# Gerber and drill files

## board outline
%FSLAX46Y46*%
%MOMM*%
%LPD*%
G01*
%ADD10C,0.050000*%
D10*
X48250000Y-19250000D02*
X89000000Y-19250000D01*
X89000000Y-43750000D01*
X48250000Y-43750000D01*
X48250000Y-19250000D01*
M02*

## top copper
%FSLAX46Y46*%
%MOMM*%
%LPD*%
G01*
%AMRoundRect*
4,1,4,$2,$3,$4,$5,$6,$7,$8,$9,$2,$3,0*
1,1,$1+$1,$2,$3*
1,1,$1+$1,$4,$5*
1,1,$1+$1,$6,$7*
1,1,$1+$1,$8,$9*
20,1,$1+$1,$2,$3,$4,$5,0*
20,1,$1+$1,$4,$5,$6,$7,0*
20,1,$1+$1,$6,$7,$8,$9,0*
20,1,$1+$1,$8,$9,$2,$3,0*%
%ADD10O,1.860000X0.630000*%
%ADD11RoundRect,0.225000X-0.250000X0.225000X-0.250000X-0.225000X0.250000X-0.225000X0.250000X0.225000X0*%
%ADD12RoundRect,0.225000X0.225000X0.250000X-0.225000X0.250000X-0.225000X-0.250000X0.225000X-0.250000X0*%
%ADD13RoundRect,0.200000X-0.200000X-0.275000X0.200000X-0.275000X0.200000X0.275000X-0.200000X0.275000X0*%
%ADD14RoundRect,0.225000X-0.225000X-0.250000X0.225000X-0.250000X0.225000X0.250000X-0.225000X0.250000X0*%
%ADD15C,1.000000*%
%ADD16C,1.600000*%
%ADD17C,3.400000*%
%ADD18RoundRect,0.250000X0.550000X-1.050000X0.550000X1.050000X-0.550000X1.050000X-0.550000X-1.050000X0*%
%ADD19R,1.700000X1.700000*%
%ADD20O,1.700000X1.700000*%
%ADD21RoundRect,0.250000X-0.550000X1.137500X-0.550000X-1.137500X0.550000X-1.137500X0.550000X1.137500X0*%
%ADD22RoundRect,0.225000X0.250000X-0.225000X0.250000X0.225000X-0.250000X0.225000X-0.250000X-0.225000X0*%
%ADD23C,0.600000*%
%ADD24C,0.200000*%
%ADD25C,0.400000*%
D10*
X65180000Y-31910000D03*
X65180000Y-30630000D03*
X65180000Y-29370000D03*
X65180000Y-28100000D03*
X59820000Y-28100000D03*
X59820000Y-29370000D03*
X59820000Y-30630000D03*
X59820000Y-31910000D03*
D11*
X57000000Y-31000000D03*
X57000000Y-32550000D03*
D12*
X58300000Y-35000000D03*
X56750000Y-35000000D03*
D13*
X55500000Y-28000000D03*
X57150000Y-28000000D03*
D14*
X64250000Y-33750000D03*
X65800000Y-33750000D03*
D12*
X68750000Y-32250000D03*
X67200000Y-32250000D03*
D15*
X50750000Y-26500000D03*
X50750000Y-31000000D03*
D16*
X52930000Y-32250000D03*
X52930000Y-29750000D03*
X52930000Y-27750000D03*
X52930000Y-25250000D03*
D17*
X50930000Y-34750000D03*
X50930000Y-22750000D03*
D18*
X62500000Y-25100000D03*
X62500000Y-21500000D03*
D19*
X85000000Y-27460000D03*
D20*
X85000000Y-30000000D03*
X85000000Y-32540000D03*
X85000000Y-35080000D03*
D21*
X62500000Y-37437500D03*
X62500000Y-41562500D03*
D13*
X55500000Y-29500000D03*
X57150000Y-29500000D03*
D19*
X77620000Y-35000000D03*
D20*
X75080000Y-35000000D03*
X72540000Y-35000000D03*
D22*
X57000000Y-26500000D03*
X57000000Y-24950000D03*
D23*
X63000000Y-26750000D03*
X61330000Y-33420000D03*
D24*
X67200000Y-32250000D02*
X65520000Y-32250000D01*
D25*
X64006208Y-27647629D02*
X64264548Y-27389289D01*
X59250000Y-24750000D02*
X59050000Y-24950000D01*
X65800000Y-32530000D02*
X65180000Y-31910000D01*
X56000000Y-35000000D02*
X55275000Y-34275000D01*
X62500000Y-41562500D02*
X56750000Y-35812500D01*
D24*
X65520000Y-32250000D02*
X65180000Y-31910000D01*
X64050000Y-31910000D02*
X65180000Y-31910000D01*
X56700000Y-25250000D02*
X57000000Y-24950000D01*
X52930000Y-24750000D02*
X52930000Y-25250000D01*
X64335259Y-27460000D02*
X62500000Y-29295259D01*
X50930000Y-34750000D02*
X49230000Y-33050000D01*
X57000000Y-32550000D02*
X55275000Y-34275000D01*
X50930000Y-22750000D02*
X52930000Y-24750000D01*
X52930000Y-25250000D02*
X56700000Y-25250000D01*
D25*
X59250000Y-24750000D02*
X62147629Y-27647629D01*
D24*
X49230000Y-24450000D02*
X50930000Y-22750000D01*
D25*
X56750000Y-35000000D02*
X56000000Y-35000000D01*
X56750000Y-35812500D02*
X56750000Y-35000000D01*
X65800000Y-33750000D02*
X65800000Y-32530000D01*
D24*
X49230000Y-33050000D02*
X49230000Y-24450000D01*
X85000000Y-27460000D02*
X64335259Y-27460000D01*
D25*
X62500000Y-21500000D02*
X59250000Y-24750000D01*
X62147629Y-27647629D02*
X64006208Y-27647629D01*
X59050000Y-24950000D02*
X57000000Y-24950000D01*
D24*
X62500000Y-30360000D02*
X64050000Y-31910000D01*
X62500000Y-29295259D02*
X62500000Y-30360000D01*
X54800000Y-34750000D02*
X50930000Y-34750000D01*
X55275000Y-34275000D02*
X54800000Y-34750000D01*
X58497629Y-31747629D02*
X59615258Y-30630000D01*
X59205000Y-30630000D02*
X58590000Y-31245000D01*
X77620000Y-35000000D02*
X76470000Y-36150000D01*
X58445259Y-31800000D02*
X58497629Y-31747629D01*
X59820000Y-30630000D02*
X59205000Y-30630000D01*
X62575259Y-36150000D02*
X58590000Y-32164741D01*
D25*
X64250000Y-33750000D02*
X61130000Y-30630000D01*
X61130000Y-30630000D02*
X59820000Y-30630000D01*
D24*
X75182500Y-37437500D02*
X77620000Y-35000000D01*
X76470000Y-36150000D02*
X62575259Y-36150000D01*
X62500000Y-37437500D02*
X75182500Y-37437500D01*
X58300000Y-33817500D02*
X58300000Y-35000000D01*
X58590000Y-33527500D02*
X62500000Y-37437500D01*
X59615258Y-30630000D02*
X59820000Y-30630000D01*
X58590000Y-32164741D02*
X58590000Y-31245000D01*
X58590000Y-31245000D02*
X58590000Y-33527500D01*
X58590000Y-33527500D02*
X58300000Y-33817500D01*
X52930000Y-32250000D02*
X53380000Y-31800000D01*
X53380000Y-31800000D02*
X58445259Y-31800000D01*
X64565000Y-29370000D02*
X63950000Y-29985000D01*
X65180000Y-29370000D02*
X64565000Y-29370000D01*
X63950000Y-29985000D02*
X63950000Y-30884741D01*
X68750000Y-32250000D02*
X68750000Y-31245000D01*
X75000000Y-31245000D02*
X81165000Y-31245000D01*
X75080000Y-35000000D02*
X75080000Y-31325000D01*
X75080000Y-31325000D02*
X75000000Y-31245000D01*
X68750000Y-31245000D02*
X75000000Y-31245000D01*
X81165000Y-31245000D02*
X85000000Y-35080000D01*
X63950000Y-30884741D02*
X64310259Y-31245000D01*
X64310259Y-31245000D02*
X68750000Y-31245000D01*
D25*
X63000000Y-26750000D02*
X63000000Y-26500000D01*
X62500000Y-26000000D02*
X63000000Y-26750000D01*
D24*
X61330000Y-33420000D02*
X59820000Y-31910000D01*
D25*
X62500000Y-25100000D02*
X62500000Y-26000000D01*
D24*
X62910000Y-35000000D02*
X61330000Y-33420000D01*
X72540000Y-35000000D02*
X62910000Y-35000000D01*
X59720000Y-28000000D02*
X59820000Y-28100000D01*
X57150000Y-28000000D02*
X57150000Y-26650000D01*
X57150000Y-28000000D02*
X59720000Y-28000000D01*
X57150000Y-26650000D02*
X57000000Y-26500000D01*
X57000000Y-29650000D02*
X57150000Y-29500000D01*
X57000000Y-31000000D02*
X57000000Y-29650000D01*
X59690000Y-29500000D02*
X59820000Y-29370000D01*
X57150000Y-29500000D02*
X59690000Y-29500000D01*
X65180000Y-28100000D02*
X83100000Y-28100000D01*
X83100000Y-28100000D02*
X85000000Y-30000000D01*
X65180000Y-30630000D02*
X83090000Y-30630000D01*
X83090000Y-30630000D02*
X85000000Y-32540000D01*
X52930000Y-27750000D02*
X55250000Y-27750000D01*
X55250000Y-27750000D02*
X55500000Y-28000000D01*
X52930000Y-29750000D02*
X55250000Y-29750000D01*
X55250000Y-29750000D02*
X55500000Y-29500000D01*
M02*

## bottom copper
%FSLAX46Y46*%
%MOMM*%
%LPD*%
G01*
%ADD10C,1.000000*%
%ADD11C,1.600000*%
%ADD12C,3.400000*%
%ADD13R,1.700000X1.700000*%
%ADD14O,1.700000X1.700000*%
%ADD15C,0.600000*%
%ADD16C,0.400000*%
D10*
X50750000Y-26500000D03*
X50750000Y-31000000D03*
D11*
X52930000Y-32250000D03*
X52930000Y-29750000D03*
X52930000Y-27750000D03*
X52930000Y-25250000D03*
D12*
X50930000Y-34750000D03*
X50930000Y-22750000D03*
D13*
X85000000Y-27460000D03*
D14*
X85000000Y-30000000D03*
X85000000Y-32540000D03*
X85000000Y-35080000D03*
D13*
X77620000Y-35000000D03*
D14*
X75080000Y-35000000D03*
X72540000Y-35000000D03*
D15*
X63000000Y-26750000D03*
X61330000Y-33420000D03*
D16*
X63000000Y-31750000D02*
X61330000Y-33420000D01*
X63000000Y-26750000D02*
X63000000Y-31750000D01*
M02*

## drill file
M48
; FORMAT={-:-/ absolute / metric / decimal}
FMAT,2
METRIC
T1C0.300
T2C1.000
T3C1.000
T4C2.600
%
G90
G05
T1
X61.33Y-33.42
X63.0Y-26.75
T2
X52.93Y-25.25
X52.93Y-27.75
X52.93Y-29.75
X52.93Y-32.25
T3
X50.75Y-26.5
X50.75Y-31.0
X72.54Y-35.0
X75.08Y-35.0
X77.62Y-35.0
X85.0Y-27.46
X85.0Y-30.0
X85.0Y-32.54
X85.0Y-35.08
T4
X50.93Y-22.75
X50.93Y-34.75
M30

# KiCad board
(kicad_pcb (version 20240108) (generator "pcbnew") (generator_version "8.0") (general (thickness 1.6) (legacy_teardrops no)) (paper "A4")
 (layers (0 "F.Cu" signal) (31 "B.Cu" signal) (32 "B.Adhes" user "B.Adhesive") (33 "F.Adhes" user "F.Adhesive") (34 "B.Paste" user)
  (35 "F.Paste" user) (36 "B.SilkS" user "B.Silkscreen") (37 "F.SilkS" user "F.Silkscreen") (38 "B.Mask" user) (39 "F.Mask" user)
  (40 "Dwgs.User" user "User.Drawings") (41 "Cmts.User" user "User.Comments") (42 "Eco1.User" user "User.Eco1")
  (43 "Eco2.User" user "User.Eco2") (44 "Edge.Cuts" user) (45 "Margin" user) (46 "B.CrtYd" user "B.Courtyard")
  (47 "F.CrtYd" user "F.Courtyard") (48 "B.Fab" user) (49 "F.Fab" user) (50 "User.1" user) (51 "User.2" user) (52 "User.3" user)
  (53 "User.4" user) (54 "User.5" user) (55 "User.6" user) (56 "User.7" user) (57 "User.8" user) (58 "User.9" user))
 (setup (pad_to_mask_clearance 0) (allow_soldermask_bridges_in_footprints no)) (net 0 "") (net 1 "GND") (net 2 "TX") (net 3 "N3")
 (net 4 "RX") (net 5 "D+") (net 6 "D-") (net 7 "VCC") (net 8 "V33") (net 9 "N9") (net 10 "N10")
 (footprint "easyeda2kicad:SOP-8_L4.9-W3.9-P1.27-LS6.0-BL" (layer "F.Cu") (at 62.5 30 90)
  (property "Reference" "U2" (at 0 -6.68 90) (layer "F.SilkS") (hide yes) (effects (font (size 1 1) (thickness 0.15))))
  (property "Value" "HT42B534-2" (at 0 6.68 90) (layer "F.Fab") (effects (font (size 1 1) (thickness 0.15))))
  (pad "1" smd oval (at -1.91 2.68 90) (size 0.63 1.86) (layers "F.Cu" "F.Paste" "F.Mask") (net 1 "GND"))
  (pad "2" smd oval (at -0.63 2.68 90) (size 0.63 1.86) (layers "F.Cu" "F.Paste" "F.Mask") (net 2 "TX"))
  (pad "3" smd oval (at 0.63 2.68 90) (size 0.63 1.86) (layers "F.Cu" "F.Paste" "F.Mask") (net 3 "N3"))
  (pad "4" smd oval (at 1.9 2.68 90) (size 0.63 1.86) (layers "F.Cu" "F.Paste" "F.Mask") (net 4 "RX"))
  (pad "5" smd oval (at 1.9 -2.68 90) (size 0.63 1.86) (layers "F.Cu" "F.Paste" "F.Mask") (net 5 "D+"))
  (pad "6" smd oval (at 0.63 -2.68 90) (size 0.63 1.86) (layers "F.Cu" "F.Paste" "F.Mask") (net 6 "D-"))
  (pad "7" smd oval (at -0.63 -2.68 90) (size 0.63 1.86) (layers "F.Cu" "F.Paste" "F.Mask") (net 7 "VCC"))
  (pad "8" smd oval (at -1.91 -2.68 90) (size 0.63 1.86) (layers "F.Cu" "F.Paste" "F.Mask") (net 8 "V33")))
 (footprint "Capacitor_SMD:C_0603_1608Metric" (layer "F.Cu") (at 57 31.775 -90)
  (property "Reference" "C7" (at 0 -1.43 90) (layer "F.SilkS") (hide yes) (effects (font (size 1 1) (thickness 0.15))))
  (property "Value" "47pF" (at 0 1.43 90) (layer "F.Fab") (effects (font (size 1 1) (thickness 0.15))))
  (pad "1" smd roundrect (at -0.775 0 270) (size 0.9 0.95) (layers "F.Cu" "F.Paste" "F.Mask") (roundrect_rratio 0.25) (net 6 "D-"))
  (pad "2" smd roundrect (at 0.775 0 270) (size 0.9 0.95) (layers "F.Cu" "F.Paste" "F.Mask") (roundrect_rratio 0.25) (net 1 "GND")))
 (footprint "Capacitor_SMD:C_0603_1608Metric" (layer "F.Cu") (at 57.525 35 180)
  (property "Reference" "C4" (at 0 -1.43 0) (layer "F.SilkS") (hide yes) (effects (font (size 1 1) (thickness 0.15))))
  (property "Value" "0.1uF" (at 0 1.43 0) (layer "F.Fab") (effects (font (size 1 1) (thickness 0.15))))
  (pad "1" smd roundrect (at -0.775 0 180) (size 0.9 0.95) (layers "F.Cu" "F.Paste" "F.Mask") (roundrect_rratio 0.25) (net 7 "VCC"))
  (pad "2" smd roundrect (at 0.775 0 180) (size 0.9 0.95) (layers "F.Cu" "F.Paste" "F.Mask") (roundrect_rratio 0.25) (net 1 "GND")))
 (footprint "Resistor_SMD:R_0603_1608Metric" (layer "F.Cu") (at 56.325 28)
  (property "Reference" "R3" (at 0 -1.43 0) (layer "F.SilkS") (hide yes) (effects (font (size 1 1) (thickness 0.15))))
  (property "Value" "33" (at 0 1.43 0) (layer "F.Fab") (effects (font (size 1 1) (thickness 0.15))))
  (pad "1" smd roundrect (at -0.825 0) (size 0.8 0.95) (layers "F.Cu" "F.Paste" "F.Mask") (roundrect_rratio 0.25) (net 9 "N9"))
  (pad "2" smd roundrect (at 0.825 0) (size 0.8 0.95) (layers "F.Cu" "F.Paste" "F.Mask") (roundrect_rratio 0.25) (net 5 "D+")))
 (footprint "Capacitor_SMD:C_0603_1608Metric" (layer "F.Cu") (at 65.025 33.75)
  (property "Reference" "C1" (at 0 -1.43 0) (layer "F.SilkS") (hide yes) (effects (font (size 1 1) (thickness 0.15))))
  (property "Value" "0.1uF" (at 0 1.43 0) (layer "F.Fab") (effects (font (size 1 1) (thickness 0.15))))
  (pad "1" smd roundrect (at -0.775 0) (size 0.9 0.95) (layers "F.Cu" "F.Paste" "F.Mask") (roundrect_rratio 0.25) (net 7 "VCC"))
  (pad "2" smd roundrect (at 0.775 0) (size 0.9 0.95) (layers "F.Cu" "F.Paste" "F.Mask") (roundrect_rratio 0.25) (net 1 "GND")))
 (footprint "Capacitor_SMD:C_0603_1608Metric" (layer "F.Cu") (at 67.975 32.25 180)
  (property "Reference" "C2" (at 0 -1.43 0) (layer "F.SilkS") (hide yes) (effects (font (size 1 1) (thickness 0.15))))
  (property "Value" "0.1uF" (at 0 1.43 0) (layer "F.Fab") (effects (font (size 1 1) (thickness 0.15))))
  (pad "1" smd roundrect (at -0.775 0 180) (size 0.9 0.95) (layers "F.Cu" "F.Paste" "F.Mask") (roundrect_rratio 0.25) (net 3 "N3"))
  (pad "2" smd roundrect (at 0.775 0 180) (size 0.9 0.95) (layers "F.Cu" "F.Paste" "F.Mask") (roundrect_rratio 0.25) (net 1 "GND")))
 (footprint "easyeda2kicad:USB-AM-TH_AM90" (layer "F.Cu") (at 51.93 28.75 -90)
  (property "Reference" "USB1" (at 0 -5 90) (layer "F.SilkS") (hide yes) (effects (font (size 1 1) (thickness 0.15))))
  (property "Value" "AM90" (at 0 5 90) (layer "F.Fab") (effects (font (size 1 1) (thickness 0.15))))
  (pad "" thru_hole circle (at -2.25 1.18 270) (size 1 1) (drill 1) (layers "*.Cu" "*.Mask") (remove_unused_layers no))
  (pad "" thru_hole circle (at 2.25 1.18 270) (size 1 1) (drill 1) (layers "*.Cu" "*.Mask") (remove_unused_layers no))
  (pad "1" thru_hole circle (at 3.5 -1 180) (size 1.6 1.6) (drill 0.999998) (layers "*.Cu" "*.Mask") (remove_unused_layers no) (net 7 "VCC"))
  (pad "2" thru_hole circle (at 1 -1 180) (size 1.6 1.6) (drill 0.999998) (layers "*.Cu" "*.Mask") (remove_unused_layers no) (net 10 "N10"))
  (pad "3" thru_hole circle (at -1 -1 180) (size 1.6 1.6) (drill 0.999998) (layers "*.Cu" "*.Mask") (remove_unused_layers no) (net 9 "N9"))
  (pad "4" thru_hole circle (at -3.5 -1 180) (size 1.6 1.6) (drill 0.999998) (layers "*.Cu" "*.Mask") (remove_unused_layers no)
   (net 1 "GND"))
  (pad "MH1" thru_hole circle (at 6 1 180) (size 3.4 3.4) (drill 2.599995) (layers "*.Cu" "*.Mask") (remove_unused_layers no) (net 1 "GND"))
  (pad "MH2" thru_hole circle (at -6 1 180) (size 3.4 3.4) (drill 2.599995) (layers "*.Cu" "*.Mask") (remove_unused_layers no) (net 1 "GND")))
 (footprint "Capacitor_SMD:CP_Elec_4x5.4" (layer "F.Cu") (at 62.5 23.3 90)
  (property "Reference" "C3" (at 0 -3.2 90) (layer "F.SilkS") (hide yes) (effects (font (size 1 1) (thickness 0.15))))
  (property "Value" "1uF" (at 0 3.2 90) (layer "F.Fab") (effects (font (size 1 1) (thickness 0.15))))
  (pad "1" smd roundrect (at -1.8 0 90) (size 2.6 1.6) (layers "F.Cu" "F.Paste" "F.Mask") (roundrect_rratio 0.15625) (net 8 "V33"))
  (pad "2" smd roundrect (at 1.8 0 90) (size 2.6 1.6) (layers "F.Cu" "F.Paste" "F.Mask") (roundrect_rratio 0.15625) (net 1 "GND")))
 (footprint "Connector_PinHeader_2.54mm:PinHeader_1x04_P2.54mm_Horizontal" (layer "F.Cu") (at 85 27.46)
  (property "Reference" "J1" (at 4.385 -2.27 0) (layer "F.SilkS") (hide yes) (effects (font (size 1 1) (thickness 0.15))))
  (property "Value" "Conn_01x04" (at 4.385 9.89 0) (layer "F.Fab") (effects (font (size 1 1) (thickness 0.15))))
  (pad "1" thru_hole rect (at 0 0) (size 1.7 1.7) (drill 1) (layers "*.Cu" "*.Mask") (remove_unused_layers no) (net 1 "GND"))
  (pad "2" thru_hole oval (at 0 2.54) (size 1.7 1.7) (drill 1) (layers "*.Cu" "*.Mask") (remove_unused_layers no) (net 4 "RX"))
  (pad "3" thru_hole oval (at 0 5.08) (size 1.7 1.7) (drill 1) (layers "*.Cu" "*.Mask") (remove_unused_layers no) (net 2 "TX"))
  (pad "4" thru_hole oval (at 0 7.62) (size 1.7 1.7) (drill 1) (layers "*.Cu" "*.Mask") (remove_unused_layers no) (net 3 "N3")))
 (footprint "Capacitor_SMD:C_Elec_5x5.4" (layer "F.Cu") (at 62.5 39.5 -90)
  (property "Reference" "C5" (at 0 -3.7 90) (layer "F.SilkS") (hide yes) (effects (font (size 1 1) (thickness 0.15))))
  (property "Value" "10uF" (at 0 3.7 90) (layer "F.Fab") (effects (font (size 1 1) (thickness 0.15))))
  (pad "1" smd roundrect (at -2.0625 0 270) (size 2.775 1.6) (layers "F.Cu" "F.Paste" "F.Mask") (roundrect_rratio 0.15625) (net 7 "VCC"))
  (pad "2" smd roundrect (at 2.0625 0 270) (size 2.775 1.6) (layers "F.Cu" "F.Paste" "F.Mask") (roundrect_rratio 0.15625) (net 1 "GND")))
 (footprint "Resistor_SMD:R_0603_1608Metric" (layer "F.Cu") (at 56.325 29.5)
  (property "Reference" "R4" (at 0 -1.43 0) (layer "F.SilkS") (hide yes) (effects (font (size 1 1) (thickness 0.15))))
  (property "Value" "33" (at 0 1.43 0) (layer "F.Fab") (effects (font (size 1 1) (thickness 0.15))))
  (pad "1" smd roundrect (at -0.825 0) (size 0.8 0.95) (layers "F.Cu" "F.Paste" "F.Mask") (roundrect_rratio 0.25) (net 10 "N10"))
  (pad "2" smd roundrect (at 0.825 0) (size 0.8 0.95) (layers "F.Cu" "F.Paste" "F.Mask") (roundrect_rratio 0.25) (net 6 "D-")))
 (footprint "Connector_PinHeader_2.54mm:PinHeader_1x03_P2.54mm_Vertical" (layer "F.Cu") (at 77.62 35 -90)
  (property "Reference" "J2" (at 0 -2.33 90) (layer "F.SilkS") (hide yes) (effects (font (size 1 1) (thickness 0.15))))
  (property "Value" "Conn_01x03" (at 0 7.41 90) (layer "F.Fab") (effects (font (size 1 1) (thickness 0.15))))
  (pad "1" thru_hole rect (at 0 0 270) (size 1.7 1.7) (drill 1) (layers "*.Cu" "*.Mask") (remove_unused_layers no) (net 7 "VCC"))
  (pad "2" thru_hole oval (at 0 2.54 270) (size 1.7 1.7) (drill 1) (layers "*.Cu" "*.Mask") (remove_unused_layers no) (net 3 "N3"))
  (pad "3" thru_hole oval (at 0 5.08 270) (size 1.7 1.7) (drill 1) (layers "*.Cu" "*.Mask") (remove_unused_layers no) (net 8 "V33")))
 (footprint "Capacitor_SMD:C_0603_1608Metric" (layer "F.Cu") (at 57 25.725 90)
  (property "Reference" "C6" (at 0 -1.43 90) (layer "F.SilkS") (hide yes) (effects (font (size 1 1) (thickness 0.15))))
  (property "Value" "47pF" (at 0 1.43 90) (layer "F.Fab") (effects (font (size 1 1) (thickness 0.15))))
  (pad "1" smd roundrect (at -0.775 0 90) (size 0.9 0.95) (layers "F.Cu" "F.Paste" "F.Mask") (roundrect_rratio 0.25) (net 5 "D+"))
  (pad "2" smd roundrect (at 0.775 0 90) (size 0.9 0.95) (layers "F.Cu" "F.Paste" "F.Mask") (roundrect_rratio 0.25) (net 1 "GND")))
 (gr_rect (start 48.25 19.25) (end 89 43.75) (stroke (width 0.05) (type default)) (fill none) (layer "Edge.Cuts"))
 (segment (start 67.2 32.25) (end 65.52 32.25) (width 0.2) (layer "F.Cu") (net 1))
 (segment (start 64.006208 27.647629) (end 64.264548 27.389289) (width 0.4) (layer "F.Cu") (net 1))
 (segment (start 59.25 24.75) (end 59.05 24.95) (width 0.4) (layer "F.Cu") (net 1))
 (segment (start 65.8 32.53) (end 65.18 31.91) (width 0.4) (layer "F.Cu") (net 1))
 (segment (start 56 35) (end 55.275 34.275) (width 0.4) (layer "F.Cu") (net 1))
 (segment (start 62.5 41.5625) (end 56.75 35.8125) (width 0.4) (layer "F.Cu") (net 1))
 (segment (start 65.52 32.25) (end 65.18 31.91) (width 0.2) (layer "F.Cu") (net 1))
 (segment (start 64.05 31.91) (end 65.18 31.91) (width 0.2) (layer "F.Cu") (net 1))
 (segment (start 56.7 25.25) (end 57 24.95) (width 0.2) (layer "F.Cu") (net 1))
 (segment (start 52.93 24.75) (end 52.93 25.25) (width 0.2) (layer "F.Cu") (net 1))
 (segment (start 64.335259 27.46) (end 62.5 29.295259) (width 0.2) (layer "F.Cu") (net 1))
 (segment (start 50.93 34.75) (end 49.23 33.05) (width 0.2) (layer "F.Cu") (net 1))
 (segment (start 57 32.55) (end 55.275 34.275) (width 0.2) (layer "F.Cu") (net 1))
 (segment (start 50.93 22.75) (end 52.93 24.75) (width 0.2) (layer "F.Cu") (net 1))
 (segment (start 52.93 25.25) (end 56.7 25.25) (width 0.2) (layer "F.Cu") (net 1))
 (segment (start 59.25 24.75) (end 62.147629 27.647629) (width 0.4) (layer "F.Cu") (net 1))
 (segment (start 49.23 24.45) (end 50.93 22.75) (width 0.2) (layer "F.Cu") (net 1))
 (segment (start 56.75 35) (end 56 35) (width 0.4) (layer "F.Cu") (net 1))
 (segment (start 56.75 35.8125) (end 56.75 35) (width 0.4) (layer "F.Cu") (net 1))
 (segment (start 65.8 33.75) (end 65.8 32.53) (width 0.4) (layer "F.Cu") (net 1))
 (segment (start 49.23 33.05) (end 49.23 24.45) (width 0.2) (layer "F.Cu") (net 1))
 (segment (start 85 27.46) (end 64.335259 27.46) (width 0.2) (layer "F.Cu") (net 1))
 (segment (start 62.5 21.5) (end 59.25 24.75) (width 0.4) (layer "F.Cu") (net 1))
 (segment (start 62.147629 27.647629) (end 64.006208 27.647629) (width 0.4) (layer "F.Cu") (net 1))
 (segment (start 59.05 24.95) (end 57 24.95) (width 0.4) (layer "F.Cu") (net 1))
 (segment (start 62.5 30.36) (end 64.05 31.91) (width 0.2) (layer "F.Cu") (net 1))
 (segment (start 62.5 29.295259) (end 62.5 30.36) (width 0.2) (layer "F.Cu") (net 1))
 (segment (start 54.8 34.75) (end 50.93 34.75) (width 0.2) (layer "F.Cu") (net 1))
 (segment (start 55.275 34.275) (end 54.8 34.75) (width 0.2) (layer "F.Cu") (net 1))
 (segment (start 58.497629 31.747629) (end 59.615258 30.63) (width 0.2) (layer "F.Cu") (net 7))
 (segment (start 59.205 30.63) (end 58.59 31.245) (width 0.2) (layer "F.Cu") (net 7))
 (segment (start 77.62 35) (end 76.47 36.15) (width 0.2) (layer "F.Cu") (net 7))
 (segment (start 58.445259 31.8) (end 58.497629 31.747629) (width 0.2) (layer "F.Cu") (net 7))
 (segment (start 59.82 30.63) (end 59.205 30.63) (width 0.2) (layer "F.Cu") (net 7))
 (segment (start 62.575259 36.15) (end 58.59 32.164741) (width 0.2) (layer "F.Cu") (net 7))
 (segment (start 64.25 33.75) (end 61.13 30.63) (width 0.4) (layer "F.Cu") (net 7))
 (segment (start 61.13 30.63) (end 59.82 30.63) (width 0.4) (layer "F.Cu") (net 7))
 (segment (start 75.1825 37.4375) (end 77.62 35) (width 0.2) (layer "F.Cu") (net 7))
 (segment (start 76.47 36.15) (end 62.575259 36.15) (width 0.2) (layer "F.Cu") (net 7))
 (segment (start 62.5 37.4375) (end 75.1825 37.4375) (width 0.2) (layer "F.Cu") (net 7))
 (segment (start 58.3 33.8175) (end 58.3 35) (width 0.2) (layer "F.Cu") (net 7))
 (segment (start 58.59 33.5275) (end 62.5 37.4375) (width 0.2) (layer "F.Cu") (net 7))
 (segment (start 59.615258 30.63) (end 59.82 30.63) (width 0.2) (layer "F.Cu") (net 7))
 (segment (start 58.59 32.164741) (end 58.59 31.245) (width 0.2) (layer "F.Cu") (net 7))
 (segment (start 58.59 31.245) (end 58.59 33.5275) (width 0.2) (layer "F.Cu") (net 7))
 (segment (start 58.59 33.5275) (end 58.3 33.8175) (width 0.2) (layer "F.Cu") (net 7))
 (segment (start 52.93 32.25) (end 53.38 31.8) (width 0.2) (layer "F.Cu") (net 7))
 (segment (start 53.38 31.8) (end 58.445259 31.8) (width 0.2) (layer "F.Cu") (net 7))
 (segment (start 64.565 29.37) (end 63.95 29.985) (width 0.2) (layer "F.Cu") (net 3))
 (segment (start 65.18 29.37) (end 64.565 29.37) (width 0.2) (layer "F.Cu") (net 3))
 (segment (start 63.95 29.985) (end 63.95 30.884741) (width 0.2) (layer "F.Cu") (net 3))
 (segment (start 68.75 32.25) (end 68.75 31.245) (width 0.2) (layer "F.Cu") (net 3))
 (segment (start 75 31.245) (end 81.165 31.245) (width 0.2) (layer "F.Cu") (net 3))
 (segment (start 75.08 35) (end 75.08 31.325) (width 0.2) (layer "F.Cu") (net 3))
 (segment (start 75.08 31.325) (end 75 31.245) (width 0.2) (layer "F.Cu") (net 3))
 (segment (start 68.75 31.245) (end 75 31.245) (width 0.2) (layer "F.Cu") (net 3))
 (segment (start 81.165 31.245) (end 85 35.08) (width 0.2) (layer "F.Cu") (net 3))
 (segment (start 63.95 30.884741) (end 64.310259 31.245) (width 0.2) (layer "F.Cu") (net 3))
 (segment (start 64.310259 31.245) (end 68.75 31.245) (width 0.2) (layer "F.Cu") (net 3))
 (segment (start 63 26.75) (end 63 26.5) (width 0.4) (layer "F.Cu") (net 8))
 (segment (start 62.5 26) (end 63 26.75) (width 0.4) (layer "F.Cu") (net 8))
 (segment (start 61.33 33.42) (end 59.82 31.91) (width 0.2) (layer "F.Cu") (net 8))
 (segment (start 62.5 25.1) (end 62.5 26) (width 0.4) (layer "F.Cu") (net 8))
 (segment (start 62.91 35) (end 61.33 33.42) (width 0.2) (layer "F.Cu") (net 8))
 (segment (start 72.54 35) (end 62.91 35) (width 0.2) (layer "F.Cu") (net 8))
 (via (at 63 26.75) (size 0.6) (drill 0.3) (layers "F.Cu" "B.Cu") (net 8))
 (via (at 61.33 33.42) (size 0.6) (drill 0.3) (layers "F.Cu" "B.Cu") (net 8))
 (segment (start 63 31.75) (end 61.33 33.42) (width 0.4) (layer "B.Cu") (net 8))
 (segment (start 63 26.75) (end 63 31.75) (width 0.4) (layer "B.Cu") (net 8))
 (segment (start 59.72 28) (end 59.82 28.1) (width 0.2) (layer "F.Cu") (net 5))
 (segment (start 57.15 28) (end 57.15 26.65) (width 0.2) (layer "F.Cu") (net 5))
 (segment (start 57.15 28) (end 59.72 28) (width 0.2) (layer "F.Cu") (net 5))
 (segment (start 57.15 26.65) (end 57 26.5) (width 0.2) (layer "F.Cu") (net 5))
 (segment (start 57 29.65) (end 57.15 29.5) (width 0.2) (layer "F.Cu") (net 6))
 (segment (start 57 31) (end 57 29.65) (width 0.2) (layer "F.Cu") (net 6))
 (segment (start 59.69 29.5) (end 59.82 29.37) (width 0.2) (layer "F.Cu") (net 6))
 (segment (start 57.15 29.5) (end 59.69 29.5) (width 0.2) (layer "F.Cu") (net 6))
 (segment (start 65.18 28.1) (end 83.1 28.1) (width 0.2) (layer "F.Cu") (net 4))
 (segment (start 83.1 28.1) (end 85 30) (width 0.2) (layer "F.Cu") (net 4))
 (segment (start 65.18 30.63) (end 83.09 30.63) (width 0.2) (layer "F.Cu") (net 2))
 (segment (start 83.09 30.63) (end 85 32.54) (width 0.2) (layer "F.Cu") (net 2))
 (segment (start 52.93 27.75) (end 55.25 27.75) (width 0.2) (layer "F.Cu") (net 9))
 (segment (start 55.25 27.75) (end 55.5 28) (width 0.2) (layer "F.Cu") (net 9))
 (segment (start 52.93 29.75) (end 55.25 29.75) (width 0.2) (layer "F.Cu") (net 10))
 (segment (start 55.25 29.75) (end 55.5 29.5) (width 0.2) (layer "F.Cu") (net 10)))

